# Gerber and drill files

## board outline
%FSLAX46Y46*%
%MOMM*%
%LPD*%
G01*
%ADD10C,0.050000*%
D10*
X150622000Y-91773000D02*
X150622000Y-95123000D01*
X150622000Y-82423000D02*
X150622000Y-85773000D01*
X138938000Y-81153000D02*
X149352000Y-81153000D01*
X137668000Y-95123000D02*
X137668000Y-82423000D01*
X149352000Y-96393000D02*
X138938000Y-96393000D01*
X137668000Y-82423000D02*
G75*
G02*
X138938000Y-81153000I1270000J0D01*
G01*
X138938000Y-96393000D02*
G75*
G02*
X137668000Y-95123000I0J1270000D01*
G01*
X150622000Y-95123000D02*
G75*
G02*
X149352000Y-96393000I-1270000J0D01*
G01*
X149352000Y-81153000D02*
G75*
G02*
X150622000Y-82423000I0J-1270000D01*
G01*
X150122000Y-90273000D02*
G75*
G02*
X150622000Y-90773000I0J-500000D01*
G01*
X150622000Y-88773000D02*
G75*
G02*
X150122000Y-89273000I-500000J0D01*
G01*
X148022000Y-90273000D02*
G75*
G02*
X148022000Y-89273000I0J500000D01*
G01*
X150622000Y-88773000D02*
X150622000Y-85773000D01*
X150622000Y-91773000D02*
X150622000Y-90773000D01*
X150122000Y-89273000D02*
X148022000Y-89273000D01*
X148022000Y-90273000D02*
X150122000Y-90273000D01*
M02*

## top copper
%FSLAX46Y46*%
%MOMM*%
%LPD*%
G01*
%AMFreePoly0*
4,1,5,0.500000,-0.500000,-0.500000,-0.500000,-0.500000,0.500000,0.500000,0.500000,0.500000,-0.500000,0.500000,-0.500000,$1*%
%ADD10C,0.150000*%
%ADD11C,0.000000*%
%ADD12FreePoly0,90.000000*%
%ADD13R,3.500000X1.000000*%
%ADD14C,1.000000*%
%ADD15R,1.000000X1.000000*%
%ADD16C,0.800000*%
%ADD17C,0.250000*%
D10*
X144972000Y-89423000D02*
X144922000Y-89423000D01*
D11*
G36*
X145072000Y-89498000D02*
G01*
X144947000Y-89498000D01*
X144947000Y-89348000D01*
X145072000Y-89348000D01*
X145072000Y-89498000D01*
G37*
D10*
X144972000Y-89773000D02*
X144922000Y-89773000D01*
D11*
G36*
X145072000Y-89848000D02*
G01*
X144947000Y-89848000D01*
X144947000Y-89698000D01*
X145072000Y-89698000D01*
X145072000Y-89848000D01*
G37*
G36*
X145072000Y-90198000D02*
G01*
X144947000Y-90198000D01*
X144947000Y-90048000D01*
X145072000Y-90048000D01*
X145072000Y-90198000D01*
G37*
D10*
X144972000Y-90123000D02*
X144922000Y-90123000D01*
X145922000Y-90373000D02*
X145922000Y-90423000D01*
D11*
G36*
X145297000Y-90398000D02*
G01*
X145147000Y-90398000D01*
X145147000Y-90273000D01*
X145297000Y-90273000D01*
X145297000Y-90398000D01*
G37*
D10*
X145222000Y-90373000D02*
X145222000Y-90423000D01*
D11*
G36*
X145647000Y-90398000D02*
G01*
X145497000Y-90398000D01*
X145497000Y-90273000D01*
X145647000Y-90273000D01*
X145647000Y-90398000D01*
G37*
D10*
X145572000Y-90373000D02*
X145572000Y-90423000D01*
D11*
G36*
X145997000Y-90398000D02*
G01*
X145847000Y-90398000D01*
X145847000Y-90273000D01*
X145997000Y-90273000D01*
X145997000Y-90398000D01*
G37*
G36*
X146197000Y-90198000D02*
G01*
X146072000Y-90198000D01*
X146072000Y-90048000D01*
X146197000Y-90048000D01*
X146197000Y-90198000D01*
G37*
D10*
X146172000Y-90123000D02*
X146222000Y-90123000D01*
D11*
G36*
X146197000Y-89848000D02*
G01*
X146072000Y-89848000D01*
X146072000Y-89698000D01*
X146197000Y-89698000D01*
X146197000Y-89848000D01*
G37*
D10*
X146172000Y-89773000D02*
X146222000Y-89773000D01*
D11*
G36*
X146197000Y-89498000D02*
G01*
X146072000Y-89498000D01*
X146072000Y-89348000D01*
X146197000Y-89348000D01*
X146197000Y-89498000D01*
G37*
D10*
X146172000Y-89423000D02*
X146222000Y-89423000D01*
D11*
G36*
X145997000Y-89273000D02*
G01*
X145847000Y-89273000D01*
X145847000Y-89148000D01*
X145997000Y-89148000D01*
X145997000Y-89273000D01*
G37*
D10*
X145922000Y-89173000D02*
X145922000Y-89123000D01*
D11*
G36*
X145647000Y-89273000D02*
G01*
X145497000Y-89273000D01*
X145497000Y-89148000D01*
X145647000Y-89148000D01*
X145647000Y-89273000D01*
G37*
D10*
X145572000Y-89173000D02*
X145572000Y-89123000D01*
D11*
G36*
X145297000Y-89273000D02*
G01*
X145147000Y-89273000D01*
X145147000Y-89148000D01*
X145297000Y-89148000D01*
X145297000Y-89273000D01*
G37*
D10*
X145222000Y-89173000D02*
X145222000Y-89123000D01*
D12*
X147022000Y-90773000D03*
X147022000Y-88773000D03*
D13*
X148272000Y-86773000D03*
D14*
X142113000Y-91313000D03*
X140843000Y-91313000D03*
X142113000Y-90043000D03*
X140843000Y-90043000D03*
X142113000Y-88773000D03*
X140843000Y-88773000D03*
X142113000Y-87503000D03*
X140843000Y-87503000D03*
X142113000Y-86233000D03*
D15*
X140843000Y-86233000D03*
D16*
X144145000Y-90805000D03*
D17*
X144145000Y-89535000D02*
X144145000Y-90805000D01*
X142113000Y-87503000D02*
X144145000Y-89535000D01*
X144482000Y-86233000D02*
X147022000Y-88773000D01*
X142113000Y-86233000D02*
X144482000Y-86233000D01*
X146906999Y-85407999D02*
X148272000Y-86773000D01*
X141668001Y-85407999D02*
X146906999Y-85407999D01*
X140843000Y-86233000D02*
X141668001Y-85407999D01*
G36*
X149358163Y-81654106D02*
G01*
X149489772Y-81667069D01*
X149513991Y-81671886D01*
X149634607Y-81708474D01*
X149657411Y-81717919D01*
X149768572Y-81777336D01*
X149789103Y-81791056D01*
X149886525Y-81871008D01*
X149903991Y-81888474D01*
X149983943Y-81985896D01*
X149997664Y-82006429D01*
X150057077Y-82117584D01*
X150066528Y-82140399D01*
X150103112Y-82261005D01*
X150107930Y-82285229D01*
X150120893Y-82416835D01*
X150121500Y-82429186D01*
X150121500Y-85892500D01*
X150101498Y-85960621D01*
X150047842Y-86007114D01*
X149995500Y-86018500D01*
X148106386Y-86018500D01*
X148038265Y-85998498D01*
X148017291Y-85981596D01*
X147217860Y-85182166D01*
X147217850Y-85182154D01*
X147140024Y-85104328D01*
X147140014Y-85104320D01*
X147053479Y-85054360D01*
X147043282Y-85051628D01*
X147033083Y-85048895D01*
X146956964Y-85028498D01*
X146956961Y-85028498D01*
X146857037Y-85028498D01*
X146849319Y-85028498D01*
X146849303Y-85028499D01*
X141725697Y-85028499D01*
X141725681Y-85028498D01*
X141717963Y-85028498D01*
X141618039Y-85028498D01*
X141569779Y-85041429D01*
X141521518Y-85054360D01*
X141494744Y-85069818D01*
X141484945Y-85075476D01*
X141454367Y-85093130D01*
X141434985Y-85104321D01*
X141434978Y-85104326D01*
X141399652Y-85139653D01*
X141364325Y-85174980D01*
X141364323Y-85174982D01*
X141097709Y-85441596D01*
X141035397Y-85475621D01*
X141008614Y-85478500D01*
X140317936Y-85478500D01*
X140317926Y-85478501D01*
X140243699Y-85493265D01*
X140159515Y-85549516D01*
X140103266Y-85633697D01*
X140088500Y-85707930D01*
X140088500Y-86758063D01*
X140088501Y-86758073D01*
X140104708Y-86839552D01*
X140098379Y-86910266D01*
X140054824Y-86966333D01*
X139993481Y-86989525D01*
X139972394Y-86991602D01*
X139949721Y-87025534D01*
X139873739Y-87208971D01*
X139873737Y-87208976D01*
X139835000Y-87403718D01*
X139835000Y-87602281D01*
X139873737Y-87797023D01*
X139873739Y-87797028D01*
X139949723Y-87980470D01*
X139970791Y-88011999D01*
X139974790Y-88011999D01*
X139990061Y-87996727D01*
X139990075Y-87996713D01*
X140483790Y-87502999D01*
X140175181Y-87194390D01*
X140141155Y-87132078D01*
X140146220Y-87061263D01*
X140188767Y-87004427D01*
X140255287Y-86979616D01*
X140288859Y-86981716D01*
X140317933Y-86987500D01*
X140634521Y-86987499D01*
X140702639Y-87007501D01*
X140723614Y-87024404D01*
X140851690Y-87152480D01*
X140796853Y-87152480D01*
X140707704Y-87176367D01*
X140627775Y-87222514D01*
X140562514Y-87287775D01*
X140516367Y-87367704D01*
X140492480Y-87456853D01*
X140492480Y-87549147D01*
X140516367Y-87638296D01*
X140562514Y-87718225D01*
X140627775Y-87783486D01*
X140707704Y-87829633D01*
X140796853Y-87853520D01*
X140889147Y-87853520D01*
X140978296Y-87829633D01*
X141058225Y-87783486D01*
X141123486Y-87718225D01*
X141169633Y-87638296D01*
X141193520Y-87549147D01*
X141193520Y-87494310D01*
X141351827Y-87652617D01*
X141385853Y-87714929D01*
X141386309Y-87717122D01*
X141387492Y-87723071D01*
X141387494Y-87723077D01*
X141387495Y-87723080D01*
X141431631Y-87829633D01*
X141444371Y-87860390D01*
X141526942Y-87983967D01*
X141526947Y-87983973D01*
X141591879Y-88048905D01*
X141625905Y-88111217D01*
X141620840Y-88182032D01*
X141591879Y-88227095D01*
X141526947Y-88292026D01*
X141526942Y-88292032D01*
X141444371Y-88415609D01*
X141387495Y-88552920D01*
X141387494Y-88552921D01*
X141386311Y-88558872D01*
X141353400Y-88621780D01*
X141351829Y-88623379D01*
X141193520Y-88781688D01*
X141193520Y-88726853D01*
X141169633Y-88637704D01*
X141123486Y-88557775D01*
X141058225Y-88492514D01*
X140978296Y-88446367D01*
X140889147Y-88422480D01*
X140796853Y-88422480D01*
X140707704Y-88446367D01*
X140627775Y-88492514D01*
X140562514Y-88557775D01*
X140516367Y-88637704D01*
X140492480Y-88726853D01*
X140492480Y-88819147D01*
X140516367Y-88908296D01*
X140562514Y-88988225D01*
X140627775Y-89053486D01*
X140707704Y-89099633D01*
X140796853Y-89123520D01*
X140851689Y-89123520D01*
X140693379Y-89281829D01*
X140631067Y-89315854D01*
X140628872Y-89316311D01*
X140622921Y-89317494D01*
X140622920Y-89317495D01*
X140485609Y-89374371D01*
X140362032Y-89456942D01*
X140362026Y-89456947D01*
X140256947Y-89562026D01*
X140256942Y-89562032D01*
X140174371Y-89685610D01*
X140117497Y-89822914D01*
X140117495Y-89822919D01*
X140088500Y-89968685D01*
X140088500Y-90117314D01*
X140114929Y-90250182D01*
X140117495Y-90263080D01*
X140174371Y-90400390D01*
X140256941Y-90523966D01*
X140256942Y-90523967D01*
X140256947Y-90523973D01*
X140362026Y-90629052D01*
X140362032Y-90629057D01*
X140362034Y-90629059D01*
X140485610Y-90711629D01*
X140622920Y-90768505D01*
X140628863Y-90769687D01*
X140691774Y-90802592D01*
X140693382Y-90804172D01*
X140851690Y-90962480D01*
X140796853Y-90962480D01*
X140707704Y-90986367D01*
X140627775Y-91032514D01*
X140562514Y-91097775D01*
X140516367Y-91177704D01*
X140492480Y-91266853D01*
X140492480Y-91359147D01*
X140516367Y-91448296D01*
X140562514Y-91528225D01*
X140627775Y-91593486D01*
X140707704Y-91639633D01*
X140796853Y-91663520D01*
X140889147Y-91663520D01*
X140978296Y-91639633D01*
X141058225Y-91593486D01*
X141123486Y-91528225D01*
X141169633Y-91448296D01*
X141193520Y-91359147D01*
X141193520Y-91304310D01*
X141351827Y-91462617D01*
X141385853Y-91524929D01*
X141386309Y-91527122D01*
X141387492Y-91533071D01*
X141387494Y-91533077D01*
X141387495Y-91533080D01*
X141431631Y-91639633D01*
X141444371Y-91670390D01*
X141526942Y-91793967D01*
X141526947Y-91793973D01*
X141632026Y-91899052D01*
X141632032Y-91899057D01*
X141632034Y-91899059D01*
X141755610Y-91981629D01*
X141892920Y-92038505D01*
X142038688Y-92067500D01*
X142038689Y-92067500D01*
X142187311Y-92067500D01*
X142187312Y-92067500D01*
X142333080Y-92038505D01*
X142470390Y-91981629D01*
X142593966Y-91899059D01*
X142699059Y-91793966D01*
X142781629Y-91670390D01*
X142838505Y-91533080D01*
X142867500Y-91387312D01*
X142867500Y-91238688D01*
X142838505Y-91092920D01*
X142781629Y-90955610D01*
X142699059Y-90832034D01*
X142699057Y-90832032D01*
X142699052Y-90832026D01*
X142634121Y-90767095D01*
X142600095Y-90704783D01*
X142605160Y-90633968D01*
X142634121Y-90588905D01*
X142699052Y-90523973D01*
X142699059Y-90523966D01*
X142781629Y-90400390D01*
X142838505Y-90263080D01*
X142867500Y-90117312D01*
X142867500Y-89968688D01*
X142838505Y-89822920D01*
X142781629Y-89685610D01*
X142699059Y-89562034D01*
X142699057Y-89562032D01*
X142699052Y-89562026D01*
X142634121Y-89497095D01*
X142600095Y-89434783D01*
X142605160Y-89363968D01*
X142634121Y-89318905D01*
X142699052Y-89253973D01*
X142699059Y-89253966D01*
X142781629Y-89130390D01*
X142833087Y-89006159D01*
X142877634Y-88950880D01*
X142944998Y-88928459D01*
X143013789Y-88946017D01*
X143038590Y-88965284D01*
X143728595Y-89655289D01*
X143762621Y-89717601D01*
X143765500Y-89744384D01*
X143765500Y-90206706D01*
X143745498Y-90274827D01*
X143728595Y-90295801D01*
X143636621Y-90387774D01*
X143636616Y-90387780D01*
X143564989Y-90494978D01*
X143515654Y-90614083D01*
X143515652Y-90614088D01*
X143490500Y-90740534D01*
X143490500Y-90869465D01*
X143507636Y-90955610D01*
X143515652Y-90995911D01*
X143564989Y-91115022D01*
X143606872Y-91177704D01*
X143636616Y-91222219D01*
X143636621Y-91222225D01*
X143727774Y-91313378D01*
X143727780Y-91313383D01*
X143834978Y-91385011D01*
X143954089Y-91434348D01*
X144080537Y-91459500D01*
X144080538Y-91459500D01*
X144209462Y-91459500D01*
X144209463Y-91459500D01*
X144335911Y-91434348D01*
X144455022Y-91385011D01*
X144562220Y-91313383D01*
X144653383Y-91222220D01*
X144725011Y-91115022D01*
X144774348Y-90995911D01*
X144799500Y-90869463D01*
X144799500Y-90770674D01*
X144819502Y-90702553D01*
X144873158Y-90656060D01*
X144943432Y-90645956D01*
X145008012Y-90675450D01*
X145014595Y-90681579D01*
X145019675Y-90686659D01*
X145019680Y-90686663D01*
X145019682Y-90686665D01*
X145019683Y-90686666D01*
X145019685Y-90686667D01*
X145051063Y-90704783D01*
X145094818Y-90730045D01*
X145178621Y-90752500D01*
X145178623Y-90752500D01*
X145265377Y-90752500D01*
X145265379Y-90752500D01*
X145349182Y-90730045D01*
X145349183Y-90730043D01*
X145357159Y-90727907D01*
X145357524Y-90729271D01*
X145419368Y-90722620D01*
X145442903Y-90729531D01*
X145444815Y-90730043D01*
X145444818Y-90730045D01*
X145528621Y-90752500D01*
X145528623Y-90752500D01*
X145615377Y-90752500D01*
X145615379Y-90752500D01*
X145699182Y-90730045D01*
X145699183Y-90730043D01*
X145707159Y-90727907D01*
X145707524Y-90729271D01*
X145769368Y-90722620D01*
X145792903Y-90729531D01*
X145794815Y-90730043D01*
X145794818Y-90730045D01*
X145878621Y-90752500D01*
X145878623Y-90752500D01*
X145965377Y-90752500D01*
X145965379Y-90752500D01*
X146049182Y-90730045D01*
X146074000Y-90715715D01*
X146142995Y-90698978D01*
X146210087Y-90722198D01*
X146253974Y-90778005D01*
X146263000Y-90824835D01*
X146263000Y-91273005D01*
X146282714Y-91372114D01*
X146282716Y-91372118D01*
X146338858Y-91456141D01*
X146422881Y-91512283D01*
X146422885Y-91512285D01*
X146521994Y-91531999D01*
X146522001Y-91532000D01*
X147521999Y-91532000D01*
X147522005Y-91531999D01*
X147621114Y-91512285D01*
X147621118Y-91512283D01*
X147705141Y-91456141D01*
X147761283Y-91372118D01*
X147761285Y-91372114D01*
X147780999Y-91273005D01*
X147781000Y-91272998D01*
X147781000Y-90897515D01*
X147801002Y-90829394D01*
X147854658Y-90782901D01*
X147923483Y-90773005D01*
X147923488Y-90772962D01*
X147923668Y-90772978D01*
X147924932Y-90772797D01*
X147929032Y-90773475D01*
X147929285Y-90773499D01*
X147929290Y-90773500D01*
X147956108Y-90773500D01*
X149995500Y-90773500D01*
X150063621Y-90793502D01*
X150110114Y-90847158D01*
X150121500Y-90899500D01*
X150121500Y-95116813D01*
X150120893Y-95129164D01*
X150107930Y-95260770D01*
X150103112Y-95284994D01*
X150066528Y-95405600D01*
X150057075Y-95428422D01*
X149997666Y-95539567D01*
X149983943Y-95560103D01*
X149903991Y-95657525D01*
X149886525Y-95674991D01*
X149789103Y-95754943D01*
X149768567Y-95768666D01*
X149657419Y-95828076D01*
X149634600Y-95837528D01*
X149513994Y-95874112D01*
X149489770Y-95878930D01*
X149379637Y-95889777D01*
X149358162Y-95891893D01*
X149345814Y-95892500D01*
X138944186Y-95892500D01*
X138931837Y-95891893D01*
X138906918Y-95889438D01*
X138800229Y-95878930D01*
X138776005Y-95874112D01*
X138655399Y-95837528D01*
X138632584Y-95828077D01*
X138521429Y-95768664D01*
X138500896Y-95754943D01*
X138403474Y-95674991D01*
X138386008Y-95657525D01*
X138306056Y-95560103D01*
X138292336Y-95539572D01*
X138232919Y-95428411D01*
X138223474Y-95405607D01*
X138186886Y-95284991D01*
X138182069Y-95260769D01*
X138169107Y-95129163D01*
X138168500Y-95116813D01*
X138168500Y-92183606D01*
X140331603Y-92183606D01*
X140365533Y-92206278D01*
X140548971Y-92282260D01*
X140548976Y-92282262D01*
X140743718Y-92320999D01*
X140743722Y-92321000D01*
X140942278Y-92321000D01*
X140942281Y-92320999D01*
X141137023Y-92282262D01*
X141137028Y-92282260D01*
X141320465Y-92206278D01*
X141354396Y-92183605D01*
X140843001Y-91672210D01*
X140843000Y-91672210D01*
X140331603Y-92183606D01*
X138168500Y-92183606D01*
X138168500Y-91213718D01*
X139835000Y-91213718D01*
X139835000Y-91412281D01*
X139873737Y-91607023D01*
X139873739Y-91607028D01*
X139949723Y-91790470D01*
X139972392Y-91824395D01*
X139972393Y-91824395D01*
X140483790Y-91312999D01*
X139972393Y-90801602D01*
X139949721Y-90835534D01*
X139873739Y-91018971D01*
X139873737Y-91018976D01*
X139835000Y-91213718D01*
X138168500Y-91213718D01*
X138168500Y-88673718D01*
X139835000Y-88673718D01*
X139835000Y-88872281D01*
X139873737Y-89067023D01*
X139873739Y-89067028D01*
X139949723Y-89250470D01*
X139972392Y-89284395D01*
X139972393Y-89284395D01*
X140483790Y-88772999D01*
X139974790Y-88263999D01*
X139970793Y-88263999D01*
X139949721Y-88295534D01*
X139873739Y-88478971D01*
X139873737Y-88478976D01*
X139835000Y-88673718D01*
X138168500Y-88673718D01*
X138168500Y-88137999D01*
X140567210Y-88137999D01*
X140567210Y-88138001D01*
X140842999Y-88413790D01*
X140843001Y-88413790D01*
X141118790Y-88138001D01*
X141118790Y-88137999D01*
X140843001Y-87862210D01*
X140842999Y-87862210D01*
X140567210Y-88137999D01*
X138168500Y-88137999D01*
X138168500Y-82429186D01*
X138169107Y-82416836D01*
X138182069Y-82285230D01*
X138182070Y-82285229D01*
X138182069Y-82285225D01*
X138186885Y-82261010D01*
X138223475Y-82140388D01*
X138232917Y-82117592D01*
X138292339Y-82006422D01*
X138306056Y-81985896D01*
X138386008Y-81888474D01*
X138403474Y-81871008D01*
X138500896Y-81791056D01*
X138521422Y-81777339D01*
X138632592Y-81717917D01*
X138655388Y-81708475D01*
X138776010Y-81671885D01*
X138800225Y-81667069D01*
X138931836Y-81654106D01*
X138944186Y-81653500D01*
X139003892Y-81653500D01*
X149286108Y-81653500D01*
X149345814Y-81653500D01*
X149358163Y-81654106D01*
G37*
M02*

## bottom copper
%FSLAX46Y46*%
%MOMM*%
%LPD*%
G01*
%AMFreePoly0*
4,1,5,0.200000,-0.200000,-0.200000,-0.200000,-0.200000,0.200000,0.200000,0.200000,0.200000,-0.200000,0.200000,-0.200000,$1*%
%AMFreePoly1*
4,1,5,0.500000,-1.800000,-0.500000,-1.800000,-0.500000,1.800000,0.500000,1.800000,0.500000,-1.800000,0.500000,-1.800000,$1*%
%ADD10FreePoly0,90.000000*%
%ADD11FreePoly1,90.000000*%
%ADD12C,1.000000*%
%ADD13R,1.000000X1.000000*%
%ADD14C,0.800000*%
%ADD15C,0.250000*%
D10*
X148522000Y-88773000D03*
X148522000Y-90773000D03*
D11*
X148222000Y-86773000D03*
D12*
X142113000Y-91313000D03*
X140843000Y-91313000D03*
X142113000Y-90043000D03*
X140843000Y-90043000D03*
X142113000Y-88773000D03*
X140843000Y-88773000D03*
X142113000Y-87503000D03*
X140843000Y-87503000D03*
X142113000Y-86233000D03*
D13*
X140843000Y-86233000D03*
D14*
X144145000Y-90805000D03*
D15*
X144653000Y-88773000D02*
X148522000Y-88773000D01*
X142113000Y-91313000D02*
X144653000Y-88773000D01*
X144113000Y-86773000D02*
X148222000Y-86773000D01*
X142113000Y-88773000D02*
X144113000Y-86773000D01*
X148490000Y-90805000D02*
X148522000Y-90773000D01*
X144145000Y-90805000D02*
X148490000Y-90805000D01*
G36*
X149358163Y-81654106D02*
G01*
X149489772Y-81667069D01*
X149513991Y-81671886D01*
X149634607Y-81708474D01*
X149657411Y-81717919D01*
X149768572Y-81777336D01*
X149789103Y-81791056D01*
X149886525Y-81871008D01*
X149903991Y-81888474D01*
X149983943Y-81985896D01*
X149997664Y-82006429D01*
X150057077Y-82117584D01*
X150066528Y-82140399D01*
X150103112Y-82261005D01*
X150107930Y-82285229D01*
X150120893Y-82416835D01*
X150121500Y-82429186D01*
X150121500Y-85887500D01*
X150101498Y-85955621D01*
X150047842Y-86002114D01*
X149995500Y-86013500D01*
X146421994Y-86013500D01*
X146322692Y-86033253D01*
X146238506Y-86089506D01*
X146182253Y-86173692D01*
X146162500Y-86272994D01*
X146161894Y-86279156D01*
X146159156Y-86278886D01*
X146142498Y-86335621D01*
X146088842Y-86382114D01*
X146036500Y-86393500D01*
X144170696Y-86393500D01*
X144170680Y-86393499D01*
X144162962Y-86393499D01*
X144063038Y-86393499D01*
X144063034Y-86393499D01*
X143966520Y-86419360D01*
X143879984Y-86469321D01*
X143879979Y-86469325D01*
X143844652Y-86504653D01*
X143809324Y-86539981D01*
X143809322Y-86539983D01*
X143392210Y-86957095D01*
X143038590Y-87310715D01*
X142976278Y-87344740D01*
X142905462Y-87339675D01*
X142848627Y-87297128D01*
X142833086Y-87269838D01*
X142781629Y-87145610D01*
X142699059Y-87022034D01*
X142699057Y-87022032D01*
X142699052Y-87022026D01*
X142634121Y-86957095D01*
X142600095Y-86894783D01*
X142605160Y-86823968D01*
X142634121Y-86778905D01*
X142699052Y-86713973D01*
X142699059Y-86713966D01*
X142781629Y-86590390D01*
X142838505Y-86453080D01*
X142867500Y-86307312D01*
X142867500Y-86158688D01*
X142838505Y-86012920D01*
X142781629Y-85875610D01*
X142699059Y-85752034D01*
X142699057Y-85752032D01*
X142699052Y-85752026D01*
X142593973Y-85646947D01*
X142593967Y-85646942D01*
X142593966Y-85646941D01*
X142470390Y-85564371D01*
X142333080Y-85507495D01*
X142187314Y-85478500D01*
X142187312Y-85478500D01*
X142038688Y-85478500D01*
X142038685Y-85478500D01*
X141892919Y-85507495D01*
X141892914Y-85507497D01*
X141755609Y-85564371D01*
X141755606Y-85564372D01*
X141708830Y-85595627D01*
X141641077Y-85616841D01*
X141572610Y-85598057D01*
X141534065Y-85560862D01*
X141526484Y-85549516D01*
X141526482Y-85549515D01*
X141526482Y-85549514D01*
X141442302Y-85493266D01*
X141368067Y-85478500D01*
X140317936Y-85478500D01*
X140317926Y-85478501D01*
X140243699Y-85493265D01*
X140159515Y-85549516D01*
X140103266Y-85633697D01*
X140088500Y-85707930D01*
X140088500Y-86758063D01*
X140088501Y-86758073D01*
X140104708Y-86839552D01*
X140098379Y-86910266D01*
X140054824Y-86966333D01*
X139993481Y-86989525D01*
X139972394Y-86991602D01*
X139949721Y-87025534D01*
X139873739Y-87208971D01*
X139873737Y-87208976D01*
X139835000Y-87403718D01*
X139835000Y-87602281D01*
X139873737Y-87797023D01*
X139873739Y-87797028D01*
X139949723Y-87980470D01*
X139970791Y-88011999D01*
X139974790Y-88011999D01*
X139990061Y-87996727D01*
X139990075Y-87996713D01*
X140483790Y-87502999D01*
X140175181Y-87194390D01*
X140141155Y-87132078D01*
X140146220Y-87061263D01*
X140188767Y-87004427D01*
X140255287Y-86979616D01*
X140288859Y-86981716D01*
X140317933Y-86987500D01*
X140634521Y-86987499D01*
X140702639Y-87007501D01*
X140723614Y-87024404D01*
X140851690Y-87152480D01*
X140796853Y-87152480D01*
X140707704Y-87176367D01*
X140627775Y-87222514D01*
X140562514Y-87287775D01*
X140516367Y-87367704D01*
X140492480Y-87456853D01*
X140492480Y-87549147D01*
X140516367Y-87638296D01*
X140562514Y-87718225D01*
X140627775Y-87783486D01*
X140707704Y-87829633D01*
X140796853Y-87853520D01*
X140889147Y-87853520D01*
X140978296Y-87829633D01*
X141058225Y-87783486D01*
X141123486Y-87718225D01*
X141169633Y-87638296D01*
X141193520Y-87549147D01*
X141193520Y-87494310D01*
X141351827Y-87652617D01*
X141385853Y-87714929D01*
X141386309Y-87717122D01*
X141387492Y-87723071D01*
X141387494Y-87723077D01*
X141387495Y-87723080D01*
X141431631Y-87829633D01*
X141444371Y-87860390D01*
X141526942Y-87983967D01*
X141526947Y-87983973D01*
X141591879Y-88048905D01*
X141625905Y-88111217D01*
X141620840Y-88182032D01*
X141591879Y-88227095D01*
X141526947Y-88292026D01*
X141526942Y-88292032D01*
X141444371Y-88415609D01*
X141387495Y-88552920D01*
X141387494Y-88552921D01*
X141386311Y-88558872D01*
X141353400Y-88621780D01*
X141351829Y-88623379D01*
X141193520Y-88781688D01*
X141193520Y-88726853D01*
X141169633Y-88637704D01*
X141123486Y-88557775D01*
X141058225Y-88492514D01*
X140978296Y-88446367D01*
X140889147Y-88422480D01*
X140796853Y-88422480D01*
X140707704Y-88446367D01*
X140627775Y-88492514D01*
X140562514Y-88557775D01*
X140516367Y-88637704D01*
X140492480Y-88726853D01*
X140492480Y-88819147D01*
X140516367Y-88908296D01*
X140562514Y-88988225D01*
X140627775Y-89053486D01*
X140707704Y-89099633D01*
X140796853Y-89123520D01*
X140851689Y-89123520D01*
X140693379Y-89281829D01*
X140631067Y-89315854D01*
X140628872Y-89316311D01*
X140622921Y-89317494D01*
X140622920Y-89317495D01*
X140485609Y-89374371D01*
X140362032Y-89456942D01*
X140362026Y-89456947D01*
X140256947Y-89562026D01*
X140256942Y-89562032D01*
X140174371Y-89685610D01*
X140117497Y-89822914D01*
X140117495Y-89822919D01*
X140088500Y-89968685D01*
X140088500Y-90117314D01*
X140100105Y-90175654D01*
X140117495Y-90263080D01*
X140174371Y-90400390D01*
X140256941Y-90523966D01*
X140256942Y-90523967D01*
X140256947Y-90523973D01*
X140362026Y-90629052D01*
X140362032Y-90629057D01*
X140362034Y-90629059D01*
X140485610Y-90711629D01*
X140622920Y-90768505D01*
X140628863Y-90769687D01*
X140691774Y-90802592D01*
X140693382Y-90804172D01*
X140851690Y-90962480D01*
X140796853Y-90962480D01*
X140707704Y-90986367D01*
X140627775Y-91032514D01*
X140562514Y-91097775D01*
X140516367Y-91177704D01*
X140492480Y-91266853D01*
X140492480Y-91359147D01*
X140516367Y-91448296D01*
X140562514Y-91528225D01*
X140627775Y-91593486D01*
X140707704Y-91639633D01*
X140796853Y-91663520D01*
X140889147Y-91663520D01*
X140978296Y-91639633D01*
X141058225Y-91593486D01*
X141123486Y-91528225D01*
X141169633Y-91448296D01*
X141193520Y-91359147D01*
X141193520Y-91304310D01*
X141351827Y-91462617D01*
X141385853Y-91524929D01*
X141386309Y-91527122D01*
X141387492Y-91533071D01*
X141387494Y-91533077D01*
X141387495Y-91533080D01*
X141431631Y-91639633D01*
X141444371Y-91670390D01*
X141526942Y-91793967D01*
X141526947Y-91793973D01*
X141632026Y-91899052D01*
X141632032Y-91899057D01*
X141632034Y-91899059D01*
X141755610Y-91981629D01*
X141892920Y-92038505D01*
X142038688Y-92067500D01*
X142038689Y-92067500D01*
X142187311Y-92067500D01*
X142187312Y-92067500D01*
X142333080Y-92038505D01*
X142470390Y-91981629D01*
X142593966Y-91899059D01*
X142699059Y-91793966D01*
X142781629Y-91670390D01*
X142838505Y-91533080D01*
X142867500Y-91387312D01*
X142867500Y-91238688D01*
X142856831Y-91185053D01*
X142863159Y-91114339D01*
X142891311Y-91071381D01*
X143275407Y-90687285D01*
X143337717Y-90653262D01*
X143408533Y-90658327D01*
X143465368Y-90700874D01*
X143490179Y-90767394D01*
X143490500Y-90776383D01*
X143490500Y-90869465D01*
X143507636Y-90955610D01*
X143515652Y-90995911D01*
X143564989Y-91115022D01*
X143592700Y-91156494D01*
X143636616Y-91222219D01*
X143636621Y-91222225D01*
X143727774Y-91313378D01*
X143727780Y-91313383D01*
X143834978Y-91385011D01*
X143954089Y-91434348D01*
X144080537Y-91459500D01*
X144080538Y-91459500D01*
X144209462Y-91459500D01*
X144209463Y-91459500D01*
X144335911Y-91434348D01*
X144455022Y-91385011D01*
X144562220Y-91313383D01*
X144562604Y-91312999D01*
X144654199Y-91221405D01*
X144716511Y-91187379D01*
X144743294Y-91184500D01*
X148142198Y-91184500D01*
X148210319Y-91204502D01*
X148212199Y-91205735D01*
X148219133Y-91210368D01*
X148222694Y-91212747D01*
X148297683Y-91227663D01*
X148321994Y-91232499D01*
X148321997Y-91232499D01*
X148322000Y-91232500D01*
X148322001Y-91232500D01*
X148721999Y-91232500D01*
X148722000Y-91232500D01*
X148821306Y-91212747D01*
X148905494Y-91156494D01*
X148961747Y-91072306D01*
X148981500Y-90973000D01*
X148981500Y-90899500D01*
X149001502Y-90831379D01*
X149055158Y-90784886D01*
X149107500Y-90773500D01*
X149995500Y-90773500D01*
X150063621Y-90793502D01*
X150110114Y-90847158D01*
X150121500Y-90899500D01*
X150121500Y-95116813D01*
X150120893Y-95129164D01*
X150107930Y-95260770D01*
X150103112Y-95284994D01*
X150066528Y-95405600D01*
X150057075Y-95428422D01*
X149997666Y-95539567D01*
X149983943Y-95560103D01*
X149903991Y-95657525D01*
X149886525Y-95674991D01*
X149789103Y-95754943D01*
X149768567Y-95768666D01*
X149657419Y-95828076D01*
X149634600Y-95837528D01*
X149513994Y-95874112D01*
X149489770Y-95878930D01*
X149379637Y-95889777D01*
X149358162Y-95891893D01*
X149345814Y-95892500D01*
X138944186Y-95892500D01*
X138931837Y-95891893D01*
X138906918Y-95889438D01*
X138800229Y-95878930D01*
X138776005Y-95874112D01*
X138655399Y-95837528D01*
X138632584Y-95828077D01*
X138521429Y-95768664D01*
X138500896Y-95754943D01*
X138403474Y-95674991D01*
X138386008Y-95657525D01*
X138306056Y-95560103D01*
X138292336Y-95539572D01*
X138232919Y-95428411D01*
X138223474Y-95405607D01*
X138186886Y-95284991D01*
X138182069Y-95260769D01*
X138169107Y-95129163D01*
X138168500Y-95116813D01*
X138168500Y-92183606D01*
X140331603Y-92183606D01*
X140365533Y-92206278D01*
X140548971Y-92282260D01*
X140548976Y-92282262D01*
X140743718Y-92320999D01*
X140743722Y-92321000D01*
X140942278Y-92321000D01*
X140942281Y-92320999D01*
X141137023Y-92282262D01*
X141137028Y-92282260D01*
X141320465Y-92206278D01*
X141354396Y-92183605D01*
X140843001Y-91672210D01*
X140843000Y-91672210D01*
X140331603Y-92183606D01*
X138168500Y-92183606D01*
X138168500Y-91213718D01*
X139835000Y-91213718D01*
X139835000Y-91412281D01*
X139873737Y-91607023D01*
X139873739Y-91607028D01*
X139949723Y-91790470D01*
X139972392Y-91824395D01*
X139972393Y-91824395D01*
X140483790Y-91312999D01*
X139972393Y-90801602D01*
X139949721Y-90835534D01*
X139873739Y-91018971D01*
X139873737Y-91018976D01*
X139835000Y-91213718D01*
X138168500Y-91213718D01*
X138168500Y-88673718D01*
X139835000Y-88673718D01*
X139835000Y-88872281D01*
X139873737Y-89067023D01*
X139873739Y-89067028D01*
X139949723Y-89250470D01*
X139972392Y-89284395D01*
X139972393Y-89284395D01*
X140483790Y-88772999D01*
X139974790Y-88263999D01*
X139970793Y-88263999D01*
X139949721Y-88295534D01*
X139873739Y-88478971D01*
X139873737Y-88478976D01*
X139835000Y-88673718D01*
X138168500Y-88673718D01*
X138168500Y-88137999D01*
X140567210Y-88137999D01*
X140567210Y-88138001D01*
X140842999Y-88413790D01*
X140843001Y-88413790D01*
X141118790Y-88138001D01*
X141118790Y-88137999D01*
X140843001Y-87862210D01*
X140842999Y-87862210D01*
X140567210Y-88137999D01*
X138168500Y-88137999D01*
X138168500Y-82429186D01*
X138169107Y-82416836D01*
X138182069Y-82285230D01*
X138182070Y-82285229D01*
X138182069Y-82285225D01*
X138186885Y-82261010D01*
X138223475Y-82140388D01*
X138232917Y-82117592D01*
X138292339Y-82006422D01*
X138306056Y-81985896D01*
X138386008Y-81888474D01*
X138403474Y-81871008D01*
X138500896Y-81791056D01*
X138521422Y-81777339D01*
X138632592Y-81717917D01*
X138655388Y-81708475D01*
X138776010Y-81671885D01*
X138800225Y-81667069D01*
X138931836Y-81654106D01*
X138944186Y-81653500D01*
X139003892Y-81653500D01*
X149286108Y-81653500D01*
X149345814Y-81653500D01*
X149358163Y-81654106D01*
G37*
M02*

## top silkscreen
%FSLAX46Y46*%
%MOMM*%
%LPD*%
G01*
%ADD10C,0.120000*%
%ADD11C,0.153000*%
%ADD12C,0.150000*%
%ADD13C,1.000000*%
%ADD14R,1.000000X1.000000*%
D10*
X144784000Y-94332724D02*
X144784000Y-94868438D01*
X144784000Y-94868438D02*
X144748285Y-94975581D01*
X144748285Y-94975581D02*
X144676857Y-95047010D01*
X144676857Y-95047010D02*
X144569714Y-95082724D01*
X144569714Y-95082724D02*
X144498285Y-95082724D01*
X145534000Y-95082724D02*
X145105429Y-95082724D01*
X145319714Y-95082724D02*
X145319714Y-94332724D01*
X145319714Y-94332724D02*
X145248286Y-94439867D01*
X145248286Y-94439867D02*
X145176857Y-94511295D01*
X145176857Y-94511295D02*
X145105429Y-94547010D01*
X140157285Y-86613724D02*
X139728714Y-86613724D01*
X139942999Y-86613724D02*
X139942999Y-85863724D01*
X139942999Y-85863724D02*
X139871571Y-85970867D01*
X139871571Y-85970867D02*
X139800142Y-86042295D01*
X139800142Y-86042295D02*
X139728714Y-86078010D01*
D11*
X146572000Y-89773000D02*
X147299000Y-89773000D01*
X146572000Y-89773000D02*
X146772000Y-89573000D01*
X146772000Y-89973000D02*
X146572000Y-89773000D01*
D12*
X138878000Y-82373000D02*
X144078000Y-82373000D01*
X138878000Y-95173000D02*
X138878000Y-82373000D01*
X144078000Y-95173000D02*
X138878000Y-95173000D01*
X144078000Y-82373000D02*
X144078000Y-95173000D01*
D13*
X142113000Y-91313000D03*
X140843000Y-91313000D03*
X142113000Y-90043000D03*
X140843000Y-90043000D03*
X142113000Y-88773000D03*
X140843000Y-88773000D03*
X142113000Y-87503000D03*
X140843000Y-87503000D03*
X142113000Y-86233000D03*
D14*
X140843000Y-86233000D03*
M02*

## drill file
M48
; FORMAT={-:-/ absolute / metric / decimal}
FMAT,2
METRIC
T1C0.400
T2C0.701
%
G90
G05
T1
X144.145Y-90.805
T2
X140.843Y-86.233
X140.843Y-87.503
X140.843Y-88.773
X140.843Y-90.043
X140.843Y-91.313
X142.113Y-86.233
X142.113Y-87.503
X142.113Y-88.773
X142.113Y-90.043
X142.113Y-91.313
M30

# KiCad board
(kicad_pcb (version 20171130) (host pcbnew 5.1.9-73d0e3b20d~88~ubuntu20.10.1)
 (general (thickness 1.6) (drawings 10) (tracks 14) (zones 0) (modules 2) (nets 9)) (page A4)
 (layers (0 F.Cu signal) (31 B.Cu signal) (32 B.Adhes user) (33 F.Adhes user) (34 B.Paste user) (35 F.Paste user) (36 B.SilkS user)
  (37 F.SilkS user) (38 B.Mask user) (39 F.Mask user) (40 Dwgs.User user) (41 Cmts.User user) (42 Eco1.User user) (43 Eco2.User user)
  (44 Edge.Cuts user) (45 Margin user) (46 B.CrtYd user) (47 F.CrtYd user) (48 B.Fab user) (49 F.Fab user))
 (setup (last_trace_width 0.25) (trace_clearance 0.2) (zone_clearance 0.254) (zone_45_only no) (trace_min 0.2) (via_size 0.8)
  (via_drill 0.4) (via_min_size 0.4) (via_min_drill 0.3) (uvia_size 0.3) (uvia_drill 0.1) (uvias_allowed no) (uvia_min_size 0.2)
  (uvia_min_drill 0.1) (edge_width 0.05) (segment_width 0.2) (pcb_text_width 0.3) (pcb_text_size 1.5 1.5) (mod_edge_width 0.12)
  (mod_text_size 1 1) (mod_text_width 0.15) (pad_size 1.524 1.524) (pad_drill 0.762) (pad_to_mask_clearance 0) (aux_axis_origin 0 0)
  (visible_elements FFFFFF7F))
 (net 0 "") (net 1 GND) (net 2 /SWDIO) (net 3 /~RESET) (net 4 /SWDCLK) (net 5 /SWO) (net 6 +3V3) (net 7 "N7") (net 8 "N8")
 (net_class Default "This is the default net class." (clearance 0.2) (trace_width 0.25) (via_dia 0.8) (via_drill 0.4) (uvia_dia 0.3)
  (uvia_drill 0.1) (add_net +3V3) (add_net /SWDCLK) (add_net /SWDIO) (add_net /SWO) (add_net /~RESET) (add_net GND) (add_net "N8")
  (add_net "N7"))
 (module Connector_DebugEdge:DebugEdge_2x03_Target (layer F.Cu) (at 150.622 88.773 90)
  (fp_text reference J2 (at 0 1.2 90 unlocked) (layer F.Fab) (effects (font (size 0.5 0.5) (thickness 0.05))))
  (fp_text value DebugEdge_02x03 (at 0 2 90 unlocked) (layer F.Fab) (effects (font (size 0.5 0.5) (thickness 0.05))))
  (fp_arc (start -2 -0.5) (end -2 0) (angle -90) (layer Edge.Cuts) (width 0.05))
  (fp_arc (start 0 -0.5) (end -0.5 -0.5) (angle -90) (layer Edge.Cuts) (width 0.05))
  (fp_arc (start -1 -2.6) (end -0.5 -2.6) (angle -180) (layer Edge.Cuts) (width 0.05))
  (fp_line (start -0.65 -5.65) (end -0.65 -5.7) (layer F.Cu) (width 0.15))
  (fp_poly (pts (xy -0.575 -5.55) (xy -0.725 -5.55) (xy -0.725 -5.675) (xy -0.575 -5.675)) (layer F.Cu) (width 0))
  (fp_line (start -1 -5.65) (end -1 -5.7) (layer F.Cu) (width 0.15))
  (fp_poly (pts (xy -0.925 -5.55) (xy -1.075 -5.55) (xy -1.075 -5.675) (xy -0.925 -5.675)) (layer F.Cu) (width 0))
  (fp_poly (pts (xy -1.275 -5.55) (xy -1.425 -5.55) (xy -1.425 -5.675) (xy -1.275 -5.675)) (layer F.Cu) (width 0))
  (fp_line (start -1.35 -5.65) (end -1.35 -5.7) (layer F.Cu) (width 0.15))
  (fp_line (start 0 0) (end 3 0) (layer Edge.Cuts) (width 0.05))
  (fp_line (start -3 0) (end -2 0) (layer Edge.Cuts) (width 0.05))
  (fp_line (start -1 -4.05) (end -1 -3.323) (layer F.SilkS) (width 0.153))
  (fp_line (start -1 -4.05) (end -0.8 -3.85) (layer F.SilkS) (width 0.153))
  (fp_line (start -1.2 -3.85) (end -1 -4.05) (layer F.SilkS) (width 0.153))
  (fp_line (start -0.5 -0.5) (end -0.5 -2.6) (layer Edge.Cuts) (width 0.05))
  (fp_line (start -1.5 -2.6) (end -1.5 -0.5) (layer Edge.Cuts) (width 0.05))
  (fp_line (start -1.6 -4.7) (end -1.65 -4.7) (layer F.Cu) (width 0.15))
  (fp_poly (pts (xy -1.5 -5.475) (xy -1.5 -5.325) (xy -1.625 -5.325) (xy -1.625 -5.475)) (layer F.Cu) (width 0))
  (fp_line (start -1.6 -5.4) (end -1.65 -5.4) (layer F.Cu) (width 0.15))
  (fp_poly (pts (xy -1.5 -5.125) (xy -1.5 -4.975) (xy -1.625 -4.975) (xy -1.625 -5.125)) (layer F.Cu) (width 0))
  (fp_line (start -1.6 -5.05) (end -1.65 -5.05) (layer F.Cu) (width 0.15))
  (fp_poly (pts (xy -1.5 -4.775) (xy -1.5 -4.625) (xy -1.625 -4.625) (xy -1.625 -4.775)) (layer F.Cu) (width 0))
  (fp_poly (pts (xy -1.425 -4.55) (xy -1.275 -4.55) (xy -1.275 -4.425) (xy -1.425 -4.425)) (layer F.Cu) (width 0))
  (fp_line (start -1.35 -4.45) (end -1.35 -4.4) (layer F.Cu) (width 0.15))
  (fp_poly (pts (xy -1.075 -4.55) (xy -0.925 -4.55) (xy -0.925 -4.425) (xy -1.075 -4.425)) (layer F.Cu) (width 0))
  (fp_line (start -1 -4.45) (end -1 -4.4) (layer F.Cu) (width 0.15))
  (fp_poly (pts (xy -0.725 -4.55) (xy -0.575 -4.55) (xy -0.575 -4.425) (xy -0.725 -4.425)) (layer F.Cu) (width 0))
  (fp_line (start -0.65 -4.45) (end -0.65 -4.4) (layer F.Cu) (width 0.15))
  (fp_poly (pts (xy -0.5 -4.625) (xy -0.5 -4.775) (xy -0.375 -4.775) (xy -0.375 -4.625)) (layer F.Cu) (width 0))
  (fp_line (start -0.4 -4.7) (end -0.35 -4.7) (layer F.Cu) (width 0.15))
  (fp_poly (pts (xy -0.5 -4.975) (xy -0.5 -5.125) (xy -0.375 -5.125) (xy -0.375 -4.975)) (layer F.Cu) (width 0))
  (fp_line (start -0.4 -5.05) (end -0.35 -5.05) (layer F.Cu) (width 0.15))
  (fp_poly (pts (xy -0.5 -5.325) (xy -0.5 -5.475) (xy -0.375 -5.475) (xy -0.375 -5.325)) (layer F.Cu) (width 0))
  (fp_line (start -0.4 -5.4) (end -0.35 -5.4) (layer F.Cu) (width 0.15))
  (pad 1 smd custom (at -2 -3.6 90) (size 1 1) (layers F.Cu F.Mask) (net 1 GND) (zone_connect 0) (options (clearance outline) (anchor rect))
   (primitives))
  (pad 2 smd custom (at 0 -3.6 90) (size 1 1) (layers F.Cu F.Mask) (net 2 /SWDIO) (zone_connect 0)
   (options (clearance outline) (anchor rect)) (primitives))
  (pad 4 smd custom (at 0 -2.1 90) (size 0.4 0.4) (layers B.Cu B.Mask) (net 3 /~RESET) (zone_connect 0)
   (options (clearance outline) (anchor rect)) (primitives))
  (pad 3 smd custom (at -2 -2.1 90) (size 0.4 0.4) (layers B.Cu B.Mask) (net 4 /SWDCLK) (zone_connect 0)
   (options (clearance outline) (anchor rect)) (primitives))
  (pad 6 smd custom (at 2 -2.4 90) (size 1 3.6) (layers B.Cu B.Mask) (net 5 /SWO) (zone_connect 0)
   (options (clearance outline) (anchor rect)) (primitives))
  (pad 5 smd rect (at 2 -2.35 270) (size 1 3.5) (layers F.Cu F.Mask) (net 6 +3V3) (zone_connect 0)))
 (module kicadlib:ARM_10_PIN (layer F.Cu) (at 141.478 88.773)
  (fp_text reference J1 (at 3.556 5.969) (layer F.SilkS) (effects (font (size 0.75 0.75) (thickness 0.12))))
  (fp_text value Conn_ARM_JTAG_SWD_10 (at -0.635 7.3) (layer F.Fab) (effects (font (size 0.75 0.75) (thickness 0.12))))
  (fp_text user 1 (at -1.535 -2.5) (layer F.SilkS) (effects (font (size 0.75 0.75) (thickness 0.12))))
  (fp_line (start -2.6 -6.4) (end 2.6 -6.4) (layer F.SilkS) (width 0.15))
  (fp_line (start -2.6 6.4) (end -2.6 -6.4) (layer F.SilkS) (width 0.15))
  (fp_line (start 2.6 6.4) (end -2.6 6.4) (layer F.SilkS) (width 0.15))
  (fp_line (start 2.6 -6.4) (end 2.6 6.4) (layer F.SilkS) (width 0.15))
  (pad 10 thru_hole circle (at 0.635 2.54) (size 1 1) (drill 0.70104) (layers *.Cu *.Mask F.SilkS) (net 3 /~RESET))
  (pad 9 thru_hole circle (at -0.635 2.54) (size 1 1) (drill 0.70104) (layers *.Cu *.Mask F.SilkS) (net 1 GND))
  (pad 8 thru_hole circle (at 0.635 1.27) (size 1 1) (drill 0.70104) (layers *.Cu *.Mask F.SilkS) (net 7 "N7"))
  (pad 7 thru_hole circle (at -0.635 1.27) (size 1 1) (drill 0.70104) (layers *.Cu *.Mask F.SilkS) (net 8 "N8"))
  (pad 6 thru_hole circle (at 0.635 0) (size 1 1) (drill 0.70104) (layers *.Cu *.Mask F.SilkS) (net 5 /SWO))
  (pad 5 thru_hole circle (at -0.635 0) (size 1 1) (drill 0.70104) (layers *.Cu *.Mask F.SilkS) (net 1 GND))
  (pad 4 thru_hole circle (at 0.635 -1.27) (size 1 1) (drill 0.70104) (layers *.Cu *.Mask F.SilkS) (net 4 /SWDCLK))
  (pad 3 thru_hole circle (at -0.635 -1.27) (size 1 1) (drill 0.70104) (layers *.Cu *.Mask F.SilkS) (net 1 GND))
  (pad 2 thru_hole circle (at 0.635 -2.54) (size 1 1) (drill 0.70104) (layers *.Cu *.Mask F.SilkS) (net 2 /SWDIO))
  (pad 1 thru_hole rect (at -0.635 -2.54) (size 1 1) (drill 0.70104) (layers *.Cu *.Mask F.SilkS) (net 6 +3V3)))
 (gr_line (start 150.622 91.773) (end 150.622 95.123) (layer Edge.Cuts) (width 0.05))
 (gr_line (start 150.622 82.423) (end 150.622 85.773) (layer Edge.Cuts) (width 0.05))
 (gr_line (start 138.938 81.153) (end 149.352 81.153) (layer Edge.Cuts) (width 0.05))
 (gr_line (start 137.668 95.123) (end 137.668 82.423) (layer Edge.Cuts) (width 0.05))
 (gr_line (start 149.352 96.393) (end 138.938 96.393) (layer Edge.Cuts) (width 0.05))
 (gr_arc (start 138.938 82.423) (end 138.938 81.153) (angle -90) (layer Edge.Cuts) (width 0.05))
 (gr_arc (start 138.938 95.123) (end 137.668 95.123) (angle -90) (layer Edge.Cuts) (width 0.05))
 (gr_arc (start 149.352 95.123) (end 149.352 96.393) (angle -90) (layer Edge.Cuts) (width 0.05))
 (gr_arc (start 149.352 82.423) (end 150.622 82.423) (angle -90) (layer Edge.Cuts) (width 0.05))
 (segment (start 144.653 88.773) (end 148.522 88.773) (width 0.25) (layer B.Cu) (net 3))
 (segment (start 142.113 91.313) (end 144.653 88.773) (width 0.25) (layer B.Cu) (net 3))
 (segment (start 144.113 86.773) (end 148.222 86.773) (width 0.25) (layer B.Cu) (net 5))
 (segment (start 142.113 88.773) (end 144.113 86.773) (width 0.25) (layer B.Cu) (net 5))
 (via (at 144.145 90.805) (size 0.8) (drill 0.4) (layers F.Cu B.Cu) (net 4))
 (segment (start 144.145 89.535) (end 144.145 90.805) (width 0.25) (layer F.Cu) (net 4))
 (segment (start 142.113 87.503) (end 144.145 89.535) (width 0.25) (layer F.Cu) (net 4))
 (segment (start 148.49 90.805) (end 148.522 90.773) (width 0.25) (layer B.Cu) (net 4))
 (segment (start 144.145 90.805) (end 148.49 90.805) (width 0.25) (layer B.Cu) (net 4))
 (segment (start 144.482 86.233) (end 147.022 88.773) (width 0.25) (layer F.Cu) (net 2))
 (segment (start 142.113 86.233) (end 144.482 86.233) (width 0.25) (layer F.Cu) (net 2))
 (segment (start 146.906999 85.407999) (end 148.272 86.773) (width 0.25) (layer F.Cu) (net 6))
 (segment (start 141.668001 85.407999) (end 146.906999 85.407999) (width 0.25) (layer F.Cu) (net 6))
 (segment (start 140.843 86.233) (end 141.668001 85.407999) (width 0.25) (layer F.Cu) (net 6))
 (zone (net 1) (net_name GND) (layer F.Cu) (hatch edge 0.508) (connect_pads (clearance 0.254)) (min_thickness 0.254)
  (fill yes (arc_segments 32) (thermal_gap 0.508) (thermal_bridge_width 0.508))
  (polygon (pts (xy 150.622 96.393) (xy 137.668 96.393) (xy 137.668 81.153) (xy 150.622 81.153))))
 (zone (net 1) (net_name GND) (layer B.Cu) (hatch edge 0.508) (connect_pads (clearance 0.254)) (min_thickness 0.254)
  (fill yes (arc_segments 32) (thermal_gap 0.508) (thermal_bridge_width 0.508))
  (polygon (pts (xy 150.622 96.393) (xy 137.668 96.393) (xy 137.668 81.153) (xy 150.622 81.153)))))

